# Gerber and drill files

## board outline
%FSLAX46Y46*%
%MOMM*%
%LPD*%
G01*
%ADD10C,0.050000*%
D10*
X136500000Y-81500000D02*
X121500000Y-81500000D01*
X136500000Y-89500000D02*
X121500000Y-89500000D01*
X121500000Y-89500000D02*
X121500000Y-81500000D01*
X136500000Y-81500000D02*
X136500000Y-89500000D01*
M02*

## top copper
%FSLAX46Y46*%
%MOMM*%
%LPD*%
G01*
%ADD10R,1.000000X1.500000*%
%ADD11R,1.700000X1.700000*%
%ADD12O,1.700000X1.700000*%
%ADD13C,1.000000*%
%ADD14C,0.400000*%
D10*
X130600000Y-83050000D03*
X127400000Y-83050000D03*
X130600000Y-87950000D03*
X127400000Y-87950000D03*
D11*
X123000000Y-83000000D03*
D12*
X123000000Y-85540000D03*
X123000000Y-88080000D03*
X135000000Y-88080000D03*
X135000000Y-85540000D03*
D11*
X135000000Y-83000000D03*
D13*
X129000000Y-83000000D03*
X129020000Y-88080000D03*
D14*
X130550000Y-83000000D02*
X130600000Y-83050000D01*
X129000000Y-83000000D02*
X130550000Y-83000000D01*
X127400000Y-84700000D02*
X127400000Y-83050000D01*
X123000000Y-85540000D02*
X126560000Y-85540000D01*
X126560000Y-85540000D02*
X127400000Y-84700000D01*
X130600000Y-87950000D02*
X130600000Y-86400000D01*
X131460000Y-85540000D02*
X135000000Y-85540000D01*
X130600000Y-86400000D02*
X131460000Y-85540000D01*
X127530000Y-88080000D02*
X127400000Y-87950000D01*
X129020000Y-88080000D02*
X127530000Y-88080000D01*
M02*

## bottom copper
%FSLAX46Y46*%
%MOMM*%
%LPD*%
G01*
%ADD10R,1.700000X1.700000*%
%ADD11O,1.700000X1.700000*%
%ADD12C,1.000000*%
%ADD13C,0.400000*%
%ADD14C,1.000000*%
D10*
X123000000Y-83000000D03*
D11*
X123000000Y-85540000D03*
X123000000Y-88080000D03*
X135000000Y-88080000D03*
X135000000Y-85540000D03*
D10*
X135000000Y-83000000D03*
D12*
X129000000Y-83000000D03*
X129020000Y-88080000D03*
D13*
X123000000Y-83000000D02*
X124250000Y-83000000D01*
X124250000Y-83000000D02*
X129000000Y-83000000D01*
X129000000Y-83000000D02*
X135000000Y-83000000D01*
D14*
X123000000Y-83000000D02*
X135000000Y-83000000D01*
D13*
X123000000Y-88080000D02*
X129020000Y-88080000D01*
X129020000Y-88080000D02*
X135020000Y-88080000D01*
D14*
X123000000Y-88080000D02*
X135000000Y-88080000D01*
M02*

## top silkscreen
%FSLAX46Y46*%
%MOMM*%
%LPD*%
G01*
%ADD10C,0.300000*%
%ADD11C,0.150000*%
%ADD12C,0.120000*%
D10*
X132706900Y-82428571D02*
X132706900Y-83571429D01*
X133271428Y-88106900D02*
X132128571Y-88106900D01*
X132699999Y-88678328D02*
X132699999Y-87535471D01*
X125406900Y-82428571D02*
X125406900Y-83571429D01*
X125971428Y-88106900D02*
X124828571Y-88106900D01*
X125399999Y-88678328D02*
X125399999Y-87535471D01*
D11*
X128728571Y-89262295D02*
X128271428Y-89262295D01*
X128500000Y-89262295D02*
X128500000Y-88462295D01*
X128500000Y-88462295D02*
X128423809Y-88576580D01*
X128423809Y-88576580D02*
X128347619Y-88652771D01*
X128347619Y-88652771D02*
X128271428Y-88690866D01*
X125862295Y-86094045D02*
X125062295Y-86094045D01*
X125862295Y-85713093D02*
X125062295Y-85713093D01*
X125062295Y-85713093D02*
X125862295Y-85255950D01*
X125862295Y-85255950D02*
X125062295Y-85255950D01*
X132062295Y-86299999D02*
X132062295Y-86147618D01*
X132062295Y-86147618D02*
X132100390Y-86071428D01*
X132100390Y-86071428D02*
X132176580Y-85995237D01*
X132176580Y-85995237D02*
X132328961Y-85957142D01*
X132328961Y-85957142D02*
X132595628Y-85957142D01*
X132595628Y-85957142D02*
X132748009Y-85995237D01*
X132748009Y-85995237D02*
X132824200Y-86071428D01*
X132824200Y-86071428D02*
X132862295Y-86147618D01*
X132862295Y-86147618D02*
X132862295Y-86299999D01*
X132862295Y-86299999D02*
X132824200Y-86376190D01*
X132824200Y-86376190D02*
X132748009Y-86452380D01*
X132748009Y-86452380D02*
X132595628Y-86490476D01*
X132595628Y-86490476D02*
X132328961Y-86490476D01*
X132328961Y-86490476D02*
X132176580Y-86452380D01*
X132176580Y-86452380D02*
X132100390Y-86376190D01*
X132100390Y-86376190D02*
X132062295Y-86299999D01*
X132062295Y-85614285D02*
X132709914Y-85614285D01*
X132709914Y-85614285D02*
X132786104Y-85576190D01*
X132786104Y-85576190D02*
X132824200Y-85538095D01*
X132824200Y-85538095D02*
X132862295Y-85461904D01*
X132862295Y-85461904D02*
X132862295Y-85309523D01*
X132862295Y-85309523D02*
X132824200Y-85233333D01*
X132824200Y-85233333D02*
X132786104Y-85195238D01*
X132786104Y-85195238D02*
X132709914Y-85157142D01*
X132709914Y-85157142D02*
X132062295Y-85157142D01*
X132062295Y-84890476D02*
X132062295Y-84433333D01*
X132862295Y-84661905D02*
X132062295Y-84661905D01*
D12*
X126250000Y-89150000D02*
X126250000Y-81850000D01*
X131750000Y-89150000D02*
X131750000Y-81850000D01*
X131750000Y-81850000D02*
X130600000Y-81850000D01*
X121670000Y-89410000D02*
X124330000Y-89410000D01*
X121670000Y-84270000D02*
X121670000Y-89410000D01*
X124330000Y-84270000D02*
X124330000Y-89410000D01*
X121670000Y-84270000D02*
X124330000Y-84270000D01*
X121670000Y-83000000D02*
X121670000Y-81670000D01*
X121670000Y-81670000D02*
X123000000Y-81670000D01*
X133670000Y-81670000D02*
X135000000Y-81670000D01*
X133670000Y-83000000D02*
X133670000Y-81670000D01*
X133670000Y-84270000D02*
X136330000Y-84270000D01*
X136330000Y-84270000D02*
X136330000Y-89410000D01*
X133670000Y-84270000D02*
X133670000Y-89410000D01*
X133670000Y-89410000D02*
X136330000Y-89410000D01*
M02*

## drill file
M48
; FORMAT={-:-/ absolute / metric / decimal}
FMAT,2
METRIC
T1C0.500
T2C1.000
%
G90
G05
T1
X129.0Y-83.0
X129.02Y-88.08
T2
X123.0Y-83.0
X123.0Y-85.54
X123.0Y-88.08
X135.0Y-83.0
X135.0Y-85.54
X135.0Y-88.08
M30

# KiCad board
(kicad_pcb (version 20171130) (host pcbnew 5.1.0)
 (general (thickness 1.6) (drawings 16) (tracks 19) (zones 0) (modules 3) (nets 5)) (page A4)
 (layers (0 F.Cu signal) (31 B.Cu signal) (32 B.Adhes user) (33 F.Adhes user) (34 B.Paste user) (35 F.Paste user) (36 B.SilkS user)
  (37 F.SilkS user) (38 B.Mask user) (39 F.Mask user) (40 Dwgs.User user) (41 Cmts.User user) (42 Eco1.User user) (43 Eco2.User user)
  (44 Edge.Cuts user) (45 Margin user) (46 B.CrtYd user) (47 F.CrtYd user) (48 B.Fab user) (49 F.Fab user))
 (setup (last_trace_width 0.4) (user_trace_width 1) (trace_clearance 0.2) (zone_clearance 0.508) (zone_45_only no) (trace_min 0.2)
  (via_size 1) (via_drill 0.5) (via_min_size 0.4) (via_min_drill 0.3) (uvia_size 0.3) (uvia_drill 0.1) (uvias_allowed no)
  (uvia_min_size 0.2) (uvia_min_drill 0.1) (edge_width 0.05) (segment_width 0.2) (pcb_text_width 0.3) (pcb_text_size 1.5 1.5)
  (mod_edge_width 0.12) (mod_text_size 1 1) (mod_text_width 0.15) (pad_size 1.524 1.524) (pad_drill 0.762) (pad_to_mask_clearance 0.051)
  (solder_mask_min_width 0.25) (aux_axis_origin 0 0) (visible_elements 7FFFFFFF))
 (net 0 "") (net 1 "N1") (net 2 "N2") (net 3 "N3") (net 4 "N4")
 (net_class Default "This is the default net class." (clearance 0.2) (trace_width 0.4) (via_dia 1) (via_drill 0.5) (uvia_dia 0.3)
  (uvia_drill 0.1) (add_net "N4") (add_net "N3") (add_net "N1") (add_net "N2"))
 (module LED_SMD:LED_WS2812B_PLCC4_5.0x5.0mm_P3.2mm (layer F.Cu) (at 129 85.5 90)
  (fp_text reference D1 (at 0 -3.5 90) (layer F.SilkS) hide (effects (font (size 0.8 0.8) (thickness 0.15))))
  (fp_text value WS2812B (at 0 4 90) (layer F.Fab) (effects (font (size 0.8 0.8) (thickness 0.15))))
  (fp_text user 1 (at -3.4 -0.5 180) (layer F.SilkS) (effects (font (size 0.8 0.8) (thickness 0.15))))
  (fp_line (start -3.65 -2.75) (end 3.65 -2.75) (layer F.SilkS) (width 0.12))
  (fp_line (start -3.65 2.75) (end 3.65 2.75) (layer F.SilkS) (width 0.12))
  (fp_line (start 3.65 2.75) (end 3.65 1.6) (layer F.SilkS) (width 0.12))
  (pad 3 smd rect (at 2.45 1.6 90) (size 1.5 1) (layers F.Cu F.Paste F.Mask) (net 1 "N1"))
  (pad 4 smd rect (at 2.45 -1.6 90) (size 1.5 1) (layers F.Cu F.Paste F.Mask) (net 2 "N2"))
  (pad 2 smd rect (at -2.45 1.6 90) (size 1.5 1) (layers F.Cu F.Paste F.Mask) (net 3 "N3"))
  (pad 1 smd rect (at -2.45 -1.6 90) (size 1.5 1) (layers F.Cu F.Paste F.Mask) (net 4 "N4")))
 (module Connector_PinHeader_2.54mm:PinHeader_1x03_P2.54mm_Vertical (layer F.Cu) (at 123 83)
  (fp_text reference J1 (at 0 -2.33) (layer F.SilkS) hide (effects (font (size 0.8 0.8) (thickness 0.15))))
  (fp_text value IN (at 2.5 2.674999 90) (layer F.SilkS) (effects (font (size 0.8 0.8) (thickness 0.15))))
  (fp_line (start -1.33 6.41) (end 1.33 6.41) (layer F.SilkS) (width 0.12))
  (fp_line (start -1.33 1.27) (end -1.33 6.41) (layer F.SilkS) (width 0.12))
  (fp_line (start 1.33 1.27) (end 1.33 6.41) (layer F.SilkS) (width 0.12))
  (fp_line (start -1.33 1.27) (end 1.33 1.27) (layer F.SilkS) (width 0.12))
  (fp_line (start -1.33 0) (end -1.33 -1.33) (layer F.SilkS) (width 0.12))
  (fp_line (start -1.33 -1.33) (end 0 -1.33) (layer F.SilkS) (width 0.12))
  (pad 1 thru_hole rect (at 0 0) (size 1.7 1.7) (drill 1) (layers *.Cu *.Mask) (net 1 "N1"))
  (pad 2 thru_hole oval (at 0 2.54) (size 1.7 1.7) (drill 1) (layers *.Cu *.Mask) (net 2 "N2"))
  (pad 3 thru_hole oval (at 0 5.08) (size 1.7 1.7) (drill 1) (layers *.Cu *.Mask) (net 4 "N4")))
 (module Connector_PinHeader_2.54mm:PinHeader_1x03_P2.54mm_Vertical (layer F.Cu) (at 135 83)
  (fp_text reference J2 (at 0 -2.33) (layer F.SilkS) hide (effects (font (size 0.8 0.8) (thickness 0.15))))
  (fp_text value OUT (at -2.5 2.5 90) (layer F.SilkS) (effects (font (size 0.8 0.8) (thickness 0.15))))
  (fp_line (start -1.33 -1.33) (end 0 -1.33) (layer F.SilkS) (width 0.12))
  (fp_line (start -1.33 0) (end -1.33 -1.33) (layer F.SilkS) (width 0.12))
  (fp_line (start -1.33 1.27) (end 1.33 1.27) (layer F.SilkS) (width 0.12))
  (fp_line (start 1.33 1.27) (end 1.33 6.41) (layer F.SilkS) (width 0.12))
  (fp_line (start -1.33 1.27) (end -1.33 6.41) (layer F.SilkS) (width 0.12))
  (fp_line (start -1.33 6.41) (end 1.33 6.41) (layer F.SilkS) (width 0.12))
  (pad 3 thru_hole oval (at 0 5.08) (size 1.7 1.7) (drill 1) (layers *.Cu *.Mask) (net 4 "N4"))
  (pad 2 thru_hole oval (at 0 2.54) (size 1.7 1.7) (drill 1) (layers *.Cu *.Mask) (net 3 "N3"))
  (pad 1 thru_hole rect (at 0 0) (size 1.7 1.7) (drill 1) (layers *.Cu *.Mask) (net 1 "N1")))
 (gr_line (start 136.5 81.5) (end 121.5 81.5) (layer Edge.Cuts) (width 0.05))
 (gr_line (start 136.5 89.5) (end 121.5 89.5) (layer Edge.Cuts) (width 0.05))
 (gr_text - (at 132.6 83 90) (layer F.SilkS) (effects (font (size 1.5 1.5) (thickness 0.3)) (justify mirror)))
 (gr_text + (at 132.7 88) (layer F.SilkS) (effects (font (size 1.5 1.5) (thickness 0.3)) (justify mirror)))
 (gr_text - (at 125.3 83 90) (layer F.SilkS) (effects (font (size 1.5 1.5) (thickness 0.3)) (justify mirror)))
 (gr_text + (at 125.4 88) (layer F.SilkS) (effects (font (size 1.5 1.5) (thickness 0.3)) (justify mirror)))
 (gr_line (start 121.5 89.5) (end 121.5 81.5) (layer Edge.Cuts) (width 0.05))
 (gr_line (start 136.5 81.5) (end 136.5 89.5) (layer Edge.Cuts) (width 0.05))
 (segment (start 123 83) (end 124.25 83) (width 0.4) (layer B.Cu) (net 1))
 (via (at 129 83) (size 1) (drill 0.5) (layers F.Cu B.Cu) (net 1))
 (segment (start 124.25 83) (end 129 83) (width 0.4) (layer B.Cu) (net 1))
 (segment (start 130.55 83) (end 130.6 83.05) (width 0.4) (layer F.Cu) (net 1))
 (segment (start 129 83) (end 130.55 83) (width 0.4) (layer F.Cu) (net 1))
 (segment (start 129 83) (end 135 83) (width 0.4) (layer B.Cu) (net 1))
 (segment (start 123 83) (end 135 83) (width 1) (layer B.Cu) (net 1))
 (segment (start 127.4 84.7) (end 127.4 83.05) (width 0.4) (layer F.Cu) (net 2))
 (segment (start 123 85.54) (end 126.56 85.54) (width 0.4) (layer F.Cu) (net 2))
 (segment (start 126.56 85.54) (end 127.4 84.7) (width 0.4) (layer F.Cu) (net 2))
 (segment (start 130.6 87.95) (end 130.6 86.4) (width 0.4) (layer F.Cu) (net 3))
 (segment (start 131.46 85.54) (end 135 85.54) (width 0.4) (layer F.Cu) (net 3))
 (segment (start 130.6 86.4) (end 131.46 85.54) (width 0.4) (layer F.Cu) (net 3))
 (via (at 129.02 88.08) (size 1) (drill 0.5) (layers F.Cu B.Cu) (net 4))
 (segment (start 123 88.08) (end 129.02 88.08) (width 0.4) (layer B.Cu) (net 4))
 (segment (start 127.53 88.08) (end 127.4 87.95) (width 0.4) (layer F.Cu) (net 4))
 (segment (start 129.02 88.08) (end 127.53 88.08) (width 0.4) (layer F.Cu) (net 4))
 (segment (start 129.02 88.08) (end 135.02 88.08) (width 0.4) (layer B.Cu) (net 4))
 (segment (start 123 88.08) (end 135 88.08) (width 1) (layer B.Cu) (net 4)))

